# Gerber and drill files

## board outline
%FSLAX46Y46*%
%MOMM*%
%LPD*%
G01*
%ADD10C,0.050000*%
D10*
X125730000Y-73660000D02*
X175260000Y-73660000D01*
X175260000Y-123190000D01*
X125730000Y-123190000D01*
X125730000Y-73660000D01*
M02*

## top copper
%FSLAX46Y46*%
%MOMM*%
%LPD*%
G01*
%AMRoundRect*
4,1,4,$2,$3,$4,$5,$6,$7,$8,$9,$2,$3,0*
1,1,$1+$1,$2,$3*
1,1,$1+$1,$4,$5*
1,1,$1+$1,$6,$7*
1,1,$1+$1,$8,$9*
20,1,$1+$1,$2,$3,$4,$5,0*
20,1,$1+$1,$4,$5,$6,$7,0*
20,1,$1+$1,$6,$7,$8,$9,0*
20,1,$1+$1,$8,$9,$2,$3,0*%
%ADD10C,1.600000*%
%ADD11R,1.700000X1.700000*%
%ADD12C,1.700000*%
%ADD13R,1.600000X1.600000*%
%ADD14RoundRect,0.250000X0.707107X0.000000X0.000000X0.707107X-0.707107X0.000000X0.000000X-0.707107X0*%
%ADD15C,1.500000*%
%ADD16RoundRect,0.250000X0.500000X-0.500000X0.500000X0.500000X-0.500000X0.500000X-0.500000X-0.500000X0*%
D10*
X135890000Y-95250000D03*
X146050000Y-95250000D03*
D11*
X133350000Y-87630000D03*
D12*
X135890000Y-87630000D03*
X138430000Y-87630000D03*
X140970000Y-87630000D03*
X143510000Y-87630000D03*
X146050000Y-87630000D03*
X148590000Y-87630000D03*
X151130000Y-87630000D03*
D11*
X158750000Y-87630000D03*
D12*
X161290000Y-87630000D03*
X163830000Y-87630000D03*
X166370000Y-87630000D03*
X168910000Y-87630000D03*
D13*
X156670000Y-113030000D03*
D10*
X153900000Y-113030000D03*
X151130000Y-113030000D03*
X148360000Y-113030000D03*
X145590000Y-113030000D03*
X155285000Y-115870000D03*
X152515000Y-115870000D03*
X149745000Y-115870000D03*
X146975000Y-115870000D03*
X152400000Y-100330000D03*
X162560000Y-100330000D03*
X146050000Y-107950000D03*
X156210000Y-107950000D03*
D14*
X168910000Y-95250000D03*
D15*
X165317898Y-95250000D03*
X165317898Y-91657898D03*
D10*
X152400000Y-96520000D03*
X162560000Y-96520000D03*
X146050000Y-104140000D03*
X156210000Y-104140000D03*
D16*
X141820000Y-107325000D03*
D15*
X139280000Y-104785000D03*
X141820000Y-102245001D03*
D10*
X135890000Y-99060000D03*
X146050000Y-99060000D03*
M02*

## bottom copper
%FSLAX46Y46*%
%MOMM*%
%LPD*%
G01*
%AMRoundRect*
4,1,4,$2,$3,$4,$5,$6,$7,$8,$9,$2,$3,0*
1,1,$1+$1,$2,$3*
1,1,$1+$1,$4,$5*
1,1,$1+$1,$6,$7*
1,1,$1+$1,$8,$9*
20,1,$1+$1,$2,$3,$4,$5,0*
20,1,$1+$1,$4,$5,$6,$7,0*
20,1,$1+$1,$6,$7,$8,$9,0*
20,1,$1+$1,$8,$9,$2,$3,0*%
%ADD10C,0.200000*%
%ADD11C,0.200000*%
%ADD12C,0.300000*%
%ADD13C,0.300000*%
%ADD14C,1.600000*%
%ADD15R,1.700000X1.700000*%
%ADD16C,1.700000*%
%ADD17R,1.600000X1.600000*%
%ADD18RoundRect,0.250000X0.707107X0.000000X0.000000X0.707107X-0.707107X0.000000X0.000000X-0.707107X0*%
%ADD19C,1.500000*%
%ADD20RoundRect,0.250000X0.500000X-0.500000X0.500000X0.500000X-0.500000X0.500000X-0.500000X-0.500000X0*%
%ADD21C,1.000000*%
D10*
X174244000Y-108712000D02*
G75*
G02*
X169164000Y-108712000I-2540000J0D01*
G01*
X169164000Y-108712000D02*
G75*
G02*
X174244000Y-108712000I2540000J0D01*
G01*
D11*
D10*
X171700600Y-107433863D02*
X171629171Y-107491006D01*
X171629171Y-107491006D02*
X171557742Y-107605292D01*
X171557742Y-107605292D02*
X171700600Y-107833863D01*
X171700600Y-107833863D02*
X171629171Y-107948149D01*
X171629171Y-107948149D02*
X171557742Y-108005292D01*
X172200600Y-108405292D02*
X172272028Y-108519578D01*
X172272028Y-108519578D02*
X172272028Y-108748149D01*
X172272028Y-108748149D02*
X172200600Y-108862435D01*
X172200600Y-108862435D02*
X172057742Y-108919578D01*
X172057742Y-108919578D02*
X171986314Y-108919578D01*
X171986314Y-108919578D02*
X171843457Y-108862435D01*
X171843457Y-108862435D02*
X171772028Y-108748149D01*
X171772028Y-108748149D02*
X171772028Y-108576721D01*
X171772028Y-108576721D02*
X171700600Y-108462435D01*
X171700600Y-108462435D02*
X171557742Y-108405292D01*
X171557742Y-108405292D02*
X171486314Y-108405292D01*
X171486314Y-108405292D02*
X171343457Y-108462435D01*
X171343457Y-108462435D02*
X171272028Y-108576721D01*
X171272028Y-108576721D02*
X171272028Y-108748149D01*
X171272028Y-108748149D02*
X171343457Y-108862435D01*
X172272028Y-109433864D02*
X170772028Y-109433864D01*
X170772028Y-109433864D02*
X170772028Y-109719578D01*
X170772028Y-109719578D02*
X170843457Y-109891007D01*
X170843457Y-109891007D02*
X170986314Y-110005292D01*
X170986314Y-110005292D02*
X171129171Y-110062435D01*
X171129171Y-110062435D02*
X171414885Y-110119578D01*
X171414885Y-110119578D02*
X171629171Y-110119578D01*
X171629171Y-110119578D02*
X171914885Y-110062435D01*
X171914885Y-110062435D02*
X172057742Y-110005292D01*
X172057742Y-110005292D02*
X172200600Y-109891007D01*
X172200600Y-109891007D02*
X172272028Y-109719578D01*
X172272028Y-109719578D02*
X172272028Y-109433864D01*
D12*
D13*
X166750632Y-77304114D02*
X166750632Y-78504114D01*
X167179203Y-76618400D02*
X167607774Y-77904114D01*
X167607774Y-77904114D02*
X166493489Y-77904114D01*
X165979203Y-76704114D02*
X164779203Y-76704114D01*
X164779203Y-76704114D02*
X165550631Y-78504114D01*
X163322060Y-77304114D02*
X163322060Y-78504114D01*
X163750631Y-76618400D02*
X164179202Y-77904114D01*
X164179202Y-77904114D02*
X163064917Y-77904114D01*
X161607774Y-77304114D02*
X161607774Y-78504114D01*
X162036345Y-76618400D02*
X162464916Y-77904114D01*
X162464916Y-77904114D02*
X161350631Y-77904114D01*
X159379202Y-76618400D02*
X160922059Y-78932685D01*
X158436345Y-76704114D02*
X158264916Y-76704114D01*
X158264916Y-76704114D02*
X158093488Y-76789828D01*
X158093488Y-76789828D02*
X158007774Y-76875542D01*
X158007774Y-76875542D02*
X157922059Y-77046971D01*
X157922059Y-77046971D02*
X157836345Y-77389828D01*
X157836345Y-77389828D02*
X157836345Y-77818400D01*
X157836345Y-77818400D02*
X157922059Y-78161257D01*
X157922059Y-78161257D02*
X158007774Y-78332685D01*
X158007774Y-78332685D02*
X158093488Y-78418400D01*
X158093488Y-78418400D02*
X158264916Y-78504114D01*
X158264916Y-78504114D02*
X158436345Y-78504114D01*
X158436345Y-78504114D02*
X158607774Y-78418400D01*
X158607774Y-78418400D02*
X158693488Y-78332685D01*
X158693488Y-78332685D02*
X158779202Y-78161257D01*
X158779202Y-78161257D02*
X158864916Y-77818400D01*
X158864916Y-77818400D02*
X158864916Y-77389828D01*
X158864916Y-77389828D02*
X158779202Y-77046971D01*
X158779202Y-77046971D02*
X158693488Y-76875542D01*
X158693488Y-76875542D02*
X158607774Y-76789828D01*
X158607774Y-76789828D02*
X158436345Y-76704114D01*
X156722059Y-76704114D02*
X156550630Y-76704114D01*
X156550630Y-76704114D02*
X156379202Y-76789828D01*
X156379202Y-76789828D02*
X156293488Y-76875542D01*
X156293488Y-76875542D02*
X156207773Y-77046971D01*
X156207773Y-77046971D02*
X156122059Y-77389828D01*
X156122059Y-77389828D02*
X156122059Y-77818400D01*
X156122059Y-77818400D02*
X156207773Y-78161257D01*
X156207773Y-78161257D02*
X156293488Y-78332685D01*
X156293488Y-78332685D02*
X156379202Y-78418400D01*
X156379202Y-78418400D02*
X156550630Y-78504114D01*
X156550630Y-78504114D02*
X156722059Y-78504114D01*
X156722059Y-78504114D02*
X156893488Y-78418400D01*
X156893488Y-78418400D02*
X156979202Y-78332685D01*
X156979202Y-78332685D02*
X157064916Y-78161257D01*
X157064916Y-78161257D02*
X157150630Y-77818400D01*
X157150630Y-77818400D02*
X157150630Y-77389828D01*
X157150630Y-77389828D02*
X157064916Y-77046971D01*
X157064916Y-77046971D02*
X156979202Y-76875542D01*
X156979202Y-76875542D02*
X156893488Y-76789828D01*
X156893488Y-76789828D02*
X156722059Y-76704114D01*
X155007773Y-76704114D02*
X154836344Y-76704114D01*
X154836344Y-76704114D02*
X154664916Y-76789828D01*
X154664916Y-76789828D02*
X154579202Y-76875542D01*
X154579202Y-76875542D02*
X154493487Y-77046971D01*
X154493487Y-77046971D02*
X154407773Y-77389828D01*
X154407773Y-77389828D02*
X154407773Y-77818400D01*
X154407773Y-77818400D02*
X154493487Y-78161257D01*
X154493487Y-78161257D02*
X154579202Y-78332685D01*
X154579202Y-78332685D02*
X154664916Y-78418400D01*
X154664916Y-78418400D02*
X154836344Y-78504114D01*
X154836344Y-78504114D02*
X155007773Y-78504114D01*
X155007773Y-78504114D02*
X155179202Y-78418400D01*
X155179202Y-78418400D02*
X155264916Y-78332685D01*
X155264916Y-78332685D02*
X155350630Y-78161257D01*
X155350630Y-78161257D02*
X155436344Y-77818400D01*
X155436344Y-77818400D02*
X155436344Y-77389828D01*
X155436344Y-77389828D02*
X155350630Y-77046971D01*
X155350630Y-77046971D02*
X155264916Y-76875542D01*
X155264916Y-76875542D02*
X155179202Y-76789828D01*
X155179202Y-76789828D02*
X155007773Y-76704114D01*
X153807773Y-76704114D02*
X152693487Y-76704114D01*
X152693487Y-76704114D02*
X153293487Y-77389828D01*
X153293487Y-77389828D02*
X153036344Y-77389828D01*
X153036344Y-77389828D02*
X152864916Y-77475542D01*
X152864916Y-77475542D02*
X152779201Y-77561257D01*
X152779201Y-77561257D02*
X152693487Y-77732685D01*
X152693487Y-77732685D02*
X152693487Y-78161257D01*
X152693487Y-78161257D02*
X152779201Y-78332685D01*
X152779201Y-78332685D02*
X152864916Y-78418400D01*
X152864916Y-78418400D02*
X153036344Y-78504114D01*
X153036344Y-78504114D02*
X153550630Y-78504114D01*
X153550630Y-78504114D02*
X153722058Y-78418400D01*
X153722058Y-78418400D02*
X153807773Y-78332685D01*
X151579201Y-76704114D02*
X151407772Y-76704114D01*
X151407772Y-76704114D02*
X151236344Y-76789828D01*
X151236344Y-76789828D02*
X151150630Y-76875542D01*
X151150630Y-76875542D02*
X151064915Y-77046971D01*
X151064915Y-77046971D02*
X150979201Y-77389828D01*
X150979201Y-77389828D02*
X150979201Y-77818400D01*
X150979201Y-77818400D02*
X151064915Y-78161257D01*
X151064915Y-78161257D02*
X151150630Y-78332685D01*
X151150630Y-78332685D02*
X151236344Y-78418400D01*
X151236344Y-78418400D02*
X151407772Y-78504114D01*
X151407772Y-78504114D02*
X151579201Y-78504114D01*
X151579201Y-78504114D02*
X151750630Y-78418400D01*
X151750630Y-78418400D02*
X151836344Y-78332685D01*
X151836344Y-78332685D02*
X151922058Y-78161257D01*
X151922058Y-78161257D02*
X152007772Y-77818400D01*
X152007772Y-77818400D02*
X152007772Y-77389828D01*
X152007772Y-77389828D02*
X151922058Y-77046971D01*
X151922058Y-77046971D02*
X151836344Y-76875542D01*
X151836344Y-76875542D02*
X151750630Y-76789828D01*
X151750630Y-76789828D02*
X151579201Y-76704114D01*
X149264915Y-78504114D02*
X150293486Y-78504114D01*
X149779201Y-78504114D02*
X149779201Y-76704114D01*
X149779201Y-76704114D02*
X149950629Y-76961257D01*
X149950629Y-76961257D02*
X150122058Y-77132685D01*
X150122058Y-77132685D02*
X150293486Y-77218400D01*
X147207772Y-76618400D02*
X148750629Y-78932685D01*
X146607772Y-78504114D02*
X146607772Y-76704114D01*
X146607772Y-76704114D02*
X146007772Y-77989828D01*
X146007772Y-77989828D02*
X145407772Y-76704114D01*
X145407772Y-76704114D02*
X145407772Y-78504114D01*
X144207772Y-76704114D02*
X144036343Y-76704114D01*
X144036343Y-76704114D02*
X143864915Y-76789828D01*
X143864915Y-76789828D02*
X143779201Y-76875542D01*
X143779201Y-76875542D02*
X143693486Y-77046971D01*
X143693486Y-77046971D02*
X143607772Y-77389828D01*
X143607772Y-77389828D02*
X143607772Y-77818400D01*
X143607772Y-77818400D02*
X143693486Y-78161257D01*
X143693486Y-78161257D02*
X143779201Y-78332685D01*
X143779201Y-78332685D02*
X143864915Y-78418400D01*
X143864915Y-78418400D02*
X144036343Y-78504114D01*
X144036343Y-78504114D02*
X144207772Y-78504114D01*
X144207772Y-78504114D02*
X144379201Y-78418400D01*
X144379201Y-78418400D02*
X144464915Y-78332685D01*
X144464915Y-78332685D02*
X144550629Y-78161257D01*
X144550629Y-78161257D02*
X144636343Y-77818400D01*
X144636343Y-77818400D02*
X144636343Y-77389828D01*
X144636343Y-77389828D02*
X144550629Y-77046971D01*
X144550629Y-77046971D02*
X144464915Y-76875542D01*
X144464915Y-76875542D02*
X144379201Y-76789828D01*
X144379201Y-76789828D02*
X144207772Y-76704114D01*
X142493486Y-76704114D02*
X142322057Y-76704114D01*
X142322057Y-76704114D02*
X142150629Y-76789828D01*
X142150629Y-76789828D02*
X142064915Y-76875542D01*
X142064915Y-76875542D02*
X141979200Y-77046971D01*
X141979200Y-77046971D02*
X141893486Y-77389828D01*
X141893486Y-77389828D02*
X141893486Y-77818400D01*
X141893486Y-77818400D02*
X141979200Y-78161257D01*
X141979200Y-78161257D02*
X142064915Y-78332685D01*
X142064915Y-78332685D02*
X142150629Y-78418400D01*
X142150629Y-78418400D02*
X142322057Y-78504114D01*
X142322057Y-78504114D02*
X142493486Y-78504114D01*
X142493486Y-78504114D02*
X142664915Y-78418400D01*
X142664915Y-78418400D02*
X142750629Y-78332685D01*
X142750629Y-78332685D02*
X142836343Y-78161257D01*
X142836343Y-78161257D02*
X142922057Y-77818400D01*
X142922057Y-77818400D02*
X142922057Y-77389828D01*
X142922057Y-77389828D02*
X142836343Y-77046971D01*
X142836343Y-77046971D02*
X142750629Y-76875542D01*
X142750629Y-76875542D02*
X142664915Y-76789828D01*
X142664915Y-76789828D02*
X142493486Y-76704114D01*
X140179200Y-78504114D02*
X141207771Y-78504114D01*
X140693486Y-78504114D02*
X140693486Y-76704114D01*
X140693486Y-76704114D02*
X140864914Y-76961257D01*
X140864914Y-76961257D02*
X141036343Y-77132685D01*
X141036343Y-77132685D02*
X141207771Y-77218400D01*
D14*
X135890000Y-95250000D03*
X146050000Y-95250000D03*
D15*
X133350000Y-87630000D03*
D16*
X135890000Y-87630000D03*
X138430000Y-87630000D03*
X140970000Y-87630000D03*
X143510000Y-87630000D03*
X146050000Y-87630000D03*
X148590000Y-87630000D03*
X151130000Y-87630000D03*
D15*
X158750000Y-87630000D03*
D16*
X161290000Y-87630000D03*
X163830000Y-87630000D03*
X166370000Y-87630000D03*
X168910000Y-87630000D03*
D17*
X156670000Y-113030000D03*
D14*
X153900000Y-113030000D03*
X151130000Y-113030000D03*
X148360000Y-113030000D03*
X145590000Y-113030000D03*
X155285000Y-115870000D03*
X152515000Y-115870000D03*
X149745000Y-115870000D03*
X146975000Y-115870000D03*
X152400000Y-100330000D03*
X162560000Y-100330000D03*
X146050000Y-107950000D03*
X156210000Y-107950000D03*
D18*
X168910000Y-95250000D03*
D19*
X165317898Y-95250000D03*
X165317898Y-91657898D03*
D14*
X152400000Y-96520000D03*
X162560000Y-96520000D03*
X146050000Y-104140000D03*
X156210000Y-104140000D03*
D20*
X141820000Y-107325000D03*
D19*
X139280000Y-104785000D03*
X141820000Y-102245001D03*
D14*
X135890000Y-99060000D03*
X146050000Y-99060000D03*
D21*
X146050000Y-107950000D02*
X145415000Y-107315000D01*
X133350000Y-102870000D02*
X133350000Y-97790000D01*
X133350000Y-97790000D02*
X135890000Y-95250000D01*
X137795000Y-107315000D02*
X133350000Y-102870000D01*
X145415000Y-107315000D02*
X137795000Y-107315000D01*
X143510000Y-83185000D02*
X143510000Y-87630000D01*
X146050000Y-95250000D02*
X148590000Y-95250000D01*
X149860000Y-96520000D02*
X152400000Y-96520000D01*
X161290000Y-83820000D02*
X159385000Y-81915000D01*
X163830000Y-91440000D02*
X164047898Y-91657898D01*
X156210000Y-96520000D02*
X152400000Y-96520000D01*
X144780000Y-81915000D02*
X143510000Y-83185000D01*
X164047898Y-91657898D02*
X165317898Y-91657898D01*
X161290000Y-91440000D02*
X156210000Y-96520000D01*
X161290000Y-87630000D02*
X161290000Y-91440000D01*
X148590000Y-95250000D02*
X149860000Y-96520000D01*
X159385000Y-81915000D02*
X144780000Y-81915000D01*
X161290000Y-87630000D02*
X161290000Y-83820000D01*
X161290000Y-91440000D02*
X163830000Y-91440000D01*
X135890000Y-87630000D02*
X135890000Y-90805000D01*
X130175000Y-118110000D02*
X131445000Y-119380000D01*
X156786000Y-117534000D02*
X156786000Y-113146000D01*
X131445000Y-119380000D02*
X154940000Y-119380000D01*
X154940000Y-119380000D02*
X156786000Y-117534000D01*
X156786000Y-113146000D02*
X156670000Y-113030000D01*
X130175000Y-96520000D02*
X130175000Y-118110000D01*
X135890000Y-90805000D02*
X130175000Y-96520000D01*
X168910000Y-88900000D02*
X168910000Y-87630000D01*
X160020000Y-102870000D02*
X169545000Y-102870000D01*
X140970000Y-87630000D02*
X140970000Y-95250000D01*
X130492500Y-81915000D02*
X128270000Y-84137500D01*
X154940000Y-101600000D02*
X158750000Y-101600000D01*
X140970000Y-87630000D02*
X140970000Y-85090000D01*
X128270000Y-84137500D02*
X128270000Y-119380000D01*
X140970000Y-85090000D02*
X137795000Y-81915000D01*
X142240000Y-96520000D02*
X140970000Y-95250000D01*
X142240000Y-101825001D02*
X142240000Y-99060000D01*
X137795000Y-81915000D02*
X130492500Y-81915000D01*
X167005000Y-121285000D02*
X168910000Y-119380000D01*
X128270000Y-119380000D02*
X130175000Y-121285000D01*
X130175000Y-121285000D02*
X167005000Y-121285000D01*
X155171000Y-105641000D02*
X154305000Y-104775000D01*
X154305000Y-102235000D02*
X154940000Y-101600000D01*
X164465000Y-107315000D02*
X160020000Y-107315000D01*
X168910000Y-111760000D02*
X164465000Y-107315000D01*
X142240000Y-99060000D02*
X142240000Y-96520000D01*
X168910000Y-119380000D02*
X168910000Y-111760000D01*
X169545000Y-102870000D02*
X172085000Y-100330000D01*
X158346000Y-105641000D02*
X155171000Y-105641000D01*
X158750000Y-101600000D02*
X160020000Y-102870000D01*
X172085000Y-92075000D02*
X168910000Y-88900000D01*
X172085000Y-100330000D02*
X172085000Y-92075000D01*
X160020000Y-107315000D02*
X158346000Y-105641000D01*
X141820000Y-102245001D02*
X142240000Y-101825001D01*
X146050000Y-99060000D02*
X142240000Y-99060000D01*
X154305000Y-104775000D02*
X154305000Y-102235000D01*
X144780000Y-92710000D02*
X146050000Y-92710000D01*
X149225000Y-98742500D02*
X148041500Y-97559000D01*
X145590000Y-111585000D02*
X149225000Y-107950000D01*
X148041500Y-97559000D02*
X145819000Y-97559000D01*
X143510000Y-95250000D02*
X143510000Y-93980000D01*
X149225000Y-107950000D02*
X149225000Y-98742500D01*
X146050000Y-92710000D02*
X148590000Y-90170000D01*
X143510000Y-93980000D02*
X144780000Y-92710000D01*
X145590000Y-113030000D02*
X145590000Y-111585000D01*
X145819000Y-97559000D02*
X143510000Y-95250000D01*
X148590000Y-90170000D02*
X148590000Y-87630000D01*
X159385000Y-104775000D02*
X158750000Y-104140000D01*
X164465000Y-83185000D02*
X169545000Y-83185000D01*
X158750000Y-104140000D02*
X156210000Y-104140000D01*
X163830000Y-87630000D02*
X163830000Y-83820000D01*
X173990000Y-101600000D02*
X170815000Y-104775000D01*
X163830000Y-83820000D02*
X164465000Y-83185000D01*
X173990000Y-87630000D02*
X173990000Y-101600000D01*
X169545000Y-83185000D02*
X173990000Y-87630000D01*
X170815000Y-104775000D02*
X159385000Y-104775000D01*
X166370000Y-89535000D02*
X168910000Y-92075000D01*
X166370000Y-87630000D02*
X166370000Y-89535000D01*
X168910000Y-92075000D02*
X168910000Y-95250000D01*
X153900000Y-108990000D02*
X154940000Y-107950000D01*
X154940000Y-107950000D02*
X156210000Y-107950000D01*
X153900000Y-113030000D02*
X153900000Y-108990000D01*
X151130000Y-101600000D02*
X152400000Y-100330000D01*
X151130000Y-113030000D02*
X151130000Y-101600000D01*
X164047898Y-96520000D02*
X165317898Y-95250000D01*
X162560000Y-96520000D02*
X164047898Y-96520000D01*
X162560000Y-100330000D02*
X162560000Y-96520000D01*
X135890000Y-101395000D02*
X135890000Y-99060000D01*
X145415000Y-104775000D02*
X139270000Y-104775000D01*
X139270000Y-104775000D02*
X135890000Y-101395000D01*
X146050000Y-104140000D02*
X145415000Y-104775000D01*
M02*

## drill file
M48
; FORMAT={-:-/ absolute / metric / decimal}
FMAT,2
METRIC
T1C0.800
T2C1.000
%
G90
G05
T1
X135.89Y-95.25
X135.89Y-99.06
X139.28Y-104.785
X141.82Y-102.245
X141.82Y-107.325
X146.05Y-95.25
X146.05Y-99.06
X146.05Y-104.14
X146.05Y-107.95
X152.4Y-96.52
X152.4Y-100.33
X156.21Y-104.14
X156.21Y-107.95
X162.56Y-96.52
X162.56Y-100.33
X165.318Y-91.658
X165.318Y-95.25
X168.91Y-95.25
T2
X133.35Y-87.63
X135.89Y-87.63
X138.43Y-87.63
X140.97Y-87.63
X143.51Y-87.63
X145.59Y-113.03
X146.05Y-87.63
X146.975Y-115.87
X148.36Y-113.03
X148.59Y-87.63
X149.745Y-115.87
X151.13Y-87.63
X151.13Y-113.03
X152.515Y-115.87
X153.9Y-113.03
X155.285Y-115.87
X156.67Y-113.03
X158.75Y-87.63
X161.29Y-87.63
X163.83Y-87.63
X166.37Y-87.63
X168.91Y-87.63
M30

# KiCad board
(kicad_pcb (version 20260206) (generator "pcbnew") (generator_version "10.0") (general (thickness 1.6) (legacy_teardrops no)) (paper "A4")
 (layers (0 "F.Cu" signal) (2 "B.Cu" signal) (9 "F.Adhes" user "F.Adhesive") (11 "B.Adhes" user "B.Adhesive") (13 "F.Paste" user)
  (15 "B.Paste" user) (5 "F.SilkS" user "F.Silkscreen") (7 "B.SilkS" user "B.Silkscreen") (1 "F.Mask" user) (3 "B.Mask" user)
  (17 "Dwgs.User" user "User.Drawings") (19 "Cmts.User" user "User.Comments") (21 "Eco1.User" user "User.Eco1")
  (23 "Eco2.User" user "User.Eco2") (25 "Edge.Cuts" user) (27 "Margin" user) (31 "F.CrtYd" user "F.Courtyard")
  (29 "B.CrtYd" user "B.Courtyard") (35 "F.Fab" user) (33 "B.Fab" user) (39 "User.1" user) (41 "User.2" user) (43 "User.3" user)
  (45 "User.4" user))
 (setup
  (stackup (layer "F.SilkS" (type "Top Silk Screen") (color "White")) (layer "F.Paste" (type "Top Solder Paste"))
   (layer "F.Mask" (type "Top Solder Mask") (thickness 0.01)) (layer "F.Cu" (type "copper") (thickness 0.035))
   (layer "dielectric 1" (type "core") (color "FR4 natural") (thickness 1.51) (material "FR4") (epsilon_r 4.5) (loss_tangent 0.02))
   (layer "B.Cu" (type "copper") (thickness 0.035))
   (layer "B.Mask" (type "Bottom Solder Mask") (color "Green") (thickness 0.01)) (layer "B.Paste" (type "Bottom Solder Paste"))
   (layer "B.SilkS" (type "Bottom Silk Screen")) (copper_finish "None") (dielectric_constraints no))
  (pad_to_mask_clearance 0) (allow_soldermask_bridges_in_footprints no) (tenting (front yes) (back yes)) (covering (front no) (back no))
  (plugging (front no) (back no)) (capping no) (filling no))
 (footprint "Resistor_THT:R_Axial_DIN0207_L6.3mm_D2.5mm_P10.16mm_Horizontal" (layer "F.Cu") (at 135.89 95.25)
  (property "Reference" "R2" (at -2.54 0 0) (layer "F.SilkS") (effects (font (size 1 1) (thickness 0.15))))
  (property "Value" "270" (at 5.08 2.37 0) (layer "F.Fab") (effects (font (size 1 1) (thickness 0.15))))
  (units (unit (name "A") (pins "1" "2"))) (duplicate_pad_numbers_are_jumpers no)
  (pad "1" thru_hole circle (at 0 0) (size 1.6 1.6) (drill 0.8) (layers "*.Cu" "*.Mask") (remove_unused_layers no) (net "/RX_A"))
  (pad "2" thru_hole circle (at 10.16 0) (size 1.6 1.6) (drill 0.8) (layers "*.Cu" "*.Mask") (remove_unused_layers no) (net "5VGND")))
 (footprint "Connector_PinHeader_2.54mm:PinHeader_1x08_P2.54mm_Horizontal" (layer "F.Cu") (at 133.35 87.63 90)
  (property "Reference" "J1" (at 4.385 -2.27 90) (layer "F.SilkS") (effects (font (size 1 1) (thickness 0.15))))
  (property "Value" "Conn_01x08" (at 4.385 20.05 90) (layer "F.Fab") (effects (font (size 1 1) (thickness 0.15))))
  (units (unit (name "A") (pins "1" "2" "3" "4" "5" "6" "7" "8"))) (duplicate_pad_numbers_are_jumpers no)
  (pad "1" thru_hole rect (at 0 0 90) (size 1.7 1.7) (drill 1) (layers "*.Cu" "*.Mask") (remove_unused_layers no) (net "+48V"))
  (pad "2" thru_hole circle (at 0 2.54 90) (size 1.7 1.7) (drill 1) (layers "*.Cu" "*.Mask") (remove_unused_layers no)
   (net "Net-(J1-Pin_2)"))
  (pad "3" thru_hole circle (at 0 5.08 90) (size 1.7 1.7) (drill 1) (layers "*.Cu" "*.Mask") (remove_unused_layers no) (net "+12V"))
  (pad "4" thru_hole circle (at 0 7.62 90) (size 1.7 1.7) (drill 1) (layers "*.Cu" "*.Mask") (remove_unused_layers no) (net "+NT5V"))
  (pad "5" thru_hole circle (at 0 10.16 90) (size 1.7 1.7) (drill 1) (layers "*.Cu" "*.Mask") (remove_unused_layers no) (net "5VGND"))
  (pad "6" thru_hole circle (at 0 12.7 90) (size 1.7 1.7) (drill 1) (layers "*.Cu" "*.Mask") (remove_unused_layers no) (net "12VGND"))
  (pad "7" thru_hole circle (at 0 15.24 90) (size 1.7 1.7) (drill 1) (layers "*.Cu" "*.Mask") (remove_unused_layers no) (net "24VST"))
  (pad "8" thru_hole circle (at 0 17.78 90) (size 1.7 1.7) (drill 1) (layers "*.Cu" "*.Mask") (remove_unused_layers no)
   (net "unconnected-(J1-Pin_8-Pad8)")))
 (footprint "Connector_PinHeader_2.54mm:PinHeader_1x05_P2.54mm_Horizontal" (layer "F.Cu") (at 158.75 87.63 90)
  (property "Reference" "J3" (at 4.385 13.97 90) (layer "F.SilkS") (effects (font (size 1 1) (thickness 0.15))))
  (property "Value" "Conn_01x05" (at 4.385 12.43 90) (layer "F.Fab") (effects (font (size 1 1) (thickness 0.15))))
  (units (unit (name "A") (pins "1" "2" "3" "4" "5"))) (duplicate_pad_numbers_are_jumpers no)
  (pad "1" thru_hole rect (at 0 0 90) (size 1.7 1.7) (drill 1) (layers "*.Cu" "*.Mask") (remove_unused_layers no)
   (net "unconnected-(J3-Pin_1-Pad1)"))
  (pad "2" thru_hole circle (at 0 2.54 90) (size 1.7 1.7) (drill 1) (layers "*.Cu" "*.Mask") (remove_unused_layers no) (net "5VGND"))
  (pad "3" thru_hole circle (at 0 5.08 90) (size 1.7 1.7) (drill 1) (layers "*.Cu" "*.Mask") (remove_unused_layers no) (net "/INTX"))
  (pad "4" thru_hole circle (at 0 7.62 90) (size 1.7 1.7) (drill 1) (layers "*.Cu" "*.Mask") (remove_unused_layers no) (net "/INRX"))
  (pad "5" thru_hole circle (at 0 10.16 90) (size 1.7 1.7) (drill 1) (layers "*.Cu" "*.Mask") (remove_unused_layers no) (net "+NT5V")))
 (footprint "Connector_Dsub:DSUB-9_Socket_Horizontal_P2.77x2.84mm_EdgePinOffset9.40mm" (layer "F.Cu") (at 156.67 113.03)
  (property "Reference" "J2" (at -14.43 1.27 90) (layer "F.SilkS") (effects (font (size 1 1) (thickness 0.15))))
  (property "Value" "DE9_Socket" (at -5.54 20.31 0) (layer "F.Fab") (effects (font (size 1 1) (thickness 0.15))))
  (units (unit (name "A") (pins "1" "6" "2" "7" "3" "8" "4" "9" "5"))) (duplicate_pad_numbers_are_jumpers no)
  (pad "1" thru_hole rect (at 0 0) (size 1.6 1.6) (drill 1) (layers "*.Cu" "*.Mask") (remove_unused_layers no) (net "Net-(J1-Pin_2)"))
  (pad "2" thru_hole circle (at -2.77 0) (size 1.6 1.6) (drill 1) (layers "*.Cu" "*.Mask") (remove_unused_layers no) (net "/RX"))
  (pad "3" thru_hole circle (at -5.54 0) (size 1.6 1.6) (drill 1) (layers "*.Cu" "*.Mask") (remove_unused_layers no) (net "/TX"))
  (pad "4" thru_hole circle (at -8.31 0) (size 1.6 1.6) (drill 1) (layers "*.Cu" "*.Mask") (remove_unused_layers no)
   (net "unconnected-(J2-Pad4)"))
  (pad "5" thru_hole circle (at -11.08 0) (size 1.6 1.6) (drill 1) (layers "*.Cu" "*.Mask") (remove_unused_layers no) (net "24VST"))
  (pad "6" thru_hole circle (at -1.385 2.84) (size 1.6 1.6) (drill 1) (layers "*.Cu" "*.Mask") (remove_unused_layers no)
   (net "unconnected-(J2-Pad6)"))
  (pad "7" thru_hole circle (at -4.155 2.84) (size 1.6 1.6) (drill 1) (layers "*.Cu" "*.Mask") (remove_unused_layers no)
   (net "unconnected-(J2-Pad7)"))
  (pad "8" thru_hole circle (at -6.925 2.84) (size 1.6 1.6) (drill 1) (layers "*.Cu" "*.Mask") (remove_unused_layers no)
   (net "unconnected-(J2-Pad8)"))
  (pad "9" thru_hole circle (at -9.695 2.84) (size 1.6 1.6) (drill 1) (layers "*.Cu" "*.Mask") (remove_unused_layers no)
   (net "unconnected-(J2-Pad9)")))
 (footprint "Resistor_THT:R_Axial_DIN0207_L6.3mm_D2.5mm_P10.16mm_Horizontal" (layer "F.Cu") (at 152.4 100.33)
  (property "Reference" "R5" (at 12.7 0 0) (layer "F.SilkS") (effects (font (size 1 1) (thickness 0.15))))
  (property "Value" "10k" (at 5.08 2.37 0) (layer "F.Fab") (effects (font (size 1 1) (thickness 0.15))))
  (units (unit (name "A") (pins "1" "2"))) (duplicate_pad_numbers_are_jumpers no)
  (pad "1" thru_hole circle (at 0 0) (size 1.6 1.6) (drill 0.8) (layers "*.Cu" "*.Mask") (remove_unused_layers no) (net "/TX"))
  (pad "2" thru_hole circle (at 10.16 0) (size 1.6 1.6) (drill 0.8) (layers "*.Cu" "*.Mask") (remove_unused_layers no) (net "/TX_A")))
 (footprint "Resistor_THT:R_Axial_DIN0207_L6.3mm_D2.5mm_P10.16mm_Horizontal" (layer "F.Cu") (at 146.05 107.95)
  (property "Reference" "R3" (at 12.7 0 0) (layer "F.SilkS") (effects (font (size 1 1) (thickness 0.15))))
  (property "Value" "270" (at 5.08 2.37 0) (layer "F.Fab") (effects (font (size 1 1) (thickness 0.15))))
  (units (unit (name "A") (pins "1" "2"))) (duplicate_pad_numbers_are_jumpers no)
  (pad "1" thru_hole circle (at 0 0) (size 1.6 1.6) (drill 0.8) (layers "*.Cu" "*.Mask") (remove_unused_layers no) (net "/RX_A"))
  (pad "2" thru_hole circle (at 10.16 0) (size 1.6 1.6) (drill 0.8) (layers "*.Cu" "*.Mask") (remove_unused_layers no) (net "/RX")))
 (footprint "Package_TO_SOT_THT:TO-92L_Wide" (layer "F.Cu") (at 168.91 95.25 135)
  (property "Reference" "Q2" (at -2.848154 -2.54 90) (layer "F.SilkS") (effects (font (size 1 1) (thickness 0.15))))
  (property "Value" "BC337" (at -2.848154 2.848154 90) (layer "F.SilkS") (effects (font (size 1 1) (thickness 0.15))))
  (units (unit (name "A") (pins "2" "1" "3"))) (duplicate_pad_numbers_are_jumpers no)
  (pad "1" thru_hole roundrect (at 0 0 135) (size 1.5 1.5) (drill 0.8) (layers "*.Cu" "*.Mask") (remove_unused_layers no)
   (roundrect_rratio 0.1666666667) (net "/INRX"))
  (pad "2" thru_hole circle (at 2.54 -2.54 135) (size 1.5 1.5) (drill 0.8) (layers "*.Cu" "*.Mask") (remove_unused_layers no) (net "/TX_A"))
  (pad "3" thru_hole circle (at 5.079999 0 135) (size 1.5 1.5) (drill 0.8) (layers "*.Cu" "*.Mask") (remove_unused_layers no) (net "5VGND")))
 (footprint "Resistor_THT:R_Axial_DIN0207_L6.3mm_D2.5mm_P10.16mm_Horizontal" (layer "F.Cu") (at 152.4 96.52)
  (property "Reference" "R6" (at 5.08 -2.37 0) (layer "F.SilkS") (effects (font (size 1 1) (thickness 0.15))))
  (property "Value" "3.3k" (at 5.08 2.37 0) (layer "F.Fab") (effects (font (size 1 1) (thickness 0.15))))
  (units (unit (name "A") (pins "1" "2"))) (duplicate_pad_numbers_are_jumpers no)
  (pad "1" thru_hole circle (at 0 0) (size 1.6 1.6) (drill 0.8) (layers "*.Cu" "*.Mask") (remove_unused_layers no) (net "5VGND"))
  (pad "2" thru_hole circle (at 10.16 0) (size 1.6 1.6) (drill 0.8) (layers "*.Cu" "*.Mask") (remove_unused_layers no) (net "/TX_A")))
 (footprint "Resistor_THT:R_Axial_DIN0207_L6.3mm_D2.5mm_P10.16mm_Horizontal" (layer "F.Cu") (at 146.05 104.14)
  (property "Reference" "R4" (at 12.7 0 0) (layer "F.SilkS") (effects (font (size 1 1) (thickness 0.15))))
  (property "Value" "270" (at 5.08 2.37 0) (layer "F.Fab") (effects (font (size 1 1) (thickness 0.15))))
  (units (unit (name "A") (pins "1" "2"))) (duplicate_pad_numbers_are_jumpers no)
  (pad "1" thru_hole circle (at 0 0) (size 1.6 1.6) (drill 0.8) (layers "*.Cu" "*.Mask") (remove_unused_layers no) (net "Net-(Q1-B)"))
  (pad "2" thru_hole circle (at 10.16 0) (size 1.6 1.6) (drill 0.8) (layers "*.Cu" "*.Mask") (remove_unused_layers no) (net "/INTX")))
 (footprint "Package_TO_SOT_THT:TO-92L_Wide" (layer "F.Cu") (at 141.82 107.325 90)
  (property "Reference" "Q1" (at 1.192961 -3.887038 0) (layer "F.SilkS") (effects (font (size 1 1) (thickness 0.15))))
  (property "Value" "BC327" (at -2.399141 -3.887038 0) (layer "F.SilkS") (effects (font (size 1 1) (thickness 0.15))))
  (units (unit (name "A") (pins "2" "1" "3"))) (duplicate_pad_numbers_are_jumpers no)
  (pad "1" thru_hole roundrect (at 0 0 90) (size 1.5 1.5) (drill 0.8) (layers "*.Cu" "*.Mask") (remove_unused_layers no)
   (roundrect_rratio 0.1666666667) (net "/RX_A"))
  (pad "2" thru_hole circle (at 2.54 -2.54 90) (size 1.5 1.5) (drill 0.8) (layers "*.Cu" "*.Mask") (remove_unused_layers no)
   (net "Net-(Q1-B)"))
  (pad "3" thru_hole circle (at 5.079999 0 90) (size 1.5 1.5) (drill 0.8) (layers "*.Cu" "*.Mask") (remove_unused_layers no) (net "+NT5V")))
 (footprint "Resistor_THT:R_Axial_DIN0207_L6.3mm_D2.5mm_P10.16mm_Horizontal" (layer "F.Cu") (at 135.89 99.06)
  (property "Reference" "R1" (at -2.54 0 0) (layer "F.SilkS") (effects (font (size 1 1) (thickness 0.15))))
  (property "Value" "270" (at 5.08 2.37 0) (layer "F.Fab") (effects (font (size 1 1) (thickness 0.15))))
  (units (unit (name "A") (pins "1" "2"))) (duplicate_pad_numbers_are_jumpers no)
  (pad "1" thru_hole circle (at 0 0) (size 1.6 1.6) (drill 0.8) (layers "*.Cu" "*.Mask") (remove_unused_layers no) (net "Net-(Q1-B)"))
  (pad "2" thru_hole circle (at 10.16 0) (size 1.6 1.6) (drill 0.8) (layers "*.Cu" "*.Mask") (remove_unused_layers no) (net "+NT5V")))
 (gr_circle (center 171.704 108.712) (end 174.244 108.712) (stroke (width 0.2) (type default)) (fill no) (layer "B.Cu"))
 (gr_rect (start 125.73 73.66) (end 175.26 123.19) (stroke (width 0.05) (type default)) (fill no) (layer "Edge.Cuts"))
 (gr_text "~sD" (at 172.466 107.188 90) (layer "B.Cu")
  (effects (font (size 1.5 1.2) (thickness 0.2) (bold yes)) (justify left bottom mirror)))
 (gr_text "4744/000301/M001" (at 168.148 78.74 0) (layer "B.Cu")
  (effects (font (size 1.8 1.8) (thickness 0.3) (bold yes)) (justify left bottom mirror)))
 (segment (start 146.05 107.95) (end 145.415 107.315) (width 1) (layer "B.Cu") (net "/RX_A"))
 (segment (start 133.35 102.87) (end 133.35 97.79) (width 1) (layer "B.Cu") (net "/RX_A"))
 (segment (start 133.35 97.79) (end 135.89 95.25) (width 1) (layer "B.Cu") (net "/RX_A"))
 (segment (start 137.795 107.315) (end 133.35 102.87) (width 1) (layer "B.Cu") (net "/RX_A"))
 (segment (start 145.415 107.315) (end 137.795 107.315) (width 1) (layer "B.Cu") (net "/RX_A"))
 (segment (start 143.51 83.185) (end 143.51 87.63) (width 1) (layer "B.Cu") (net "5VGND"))
 (segment (start 146.05 95.25) (end 148.59 95.25) (width 1) (layer "B.Cu") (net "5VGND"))
 (segment (start 149.86 96.52) (end 152.4 96.52) (width 1) (layer "B.Cu") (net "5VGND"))
 (segment (start 161.29 83.82) (end 159.385 81.915) (width 1) (layer "B.Cu") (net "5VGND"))
 (segment (start 163.83 91.44) (end 164.047898 91.657898) (width 1) (layer "B.Cu") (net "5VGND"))
 (segment (start 156.21 96.52) (end 152.4 96.52) (width 1) (layer "B.Cu") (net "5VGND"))
 (segment (start 144.78 81.915) (end 143.51 83.185) (width 1) (layer "B.Cu") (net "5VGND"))
 (segment (start 164.047898 91.657898) (end 165.317898 91.657898) (width 1) (layer "B.Cu") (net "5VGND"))
 (segment (start 161.29 91.44) (end 156.21 96.52) (width 1) (layer "B.Cu") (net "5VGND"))
 (segment (start 161.29 87.63) (end 161.29 91.44) (width 1) (layer "B.Cu") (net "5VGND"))
 (segment (start 148.59 95.25) (end 149.86 96.52) (width 1) (layer "B.Cu") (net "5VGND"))
 (segment (start 159.385 81.915) (end 144.78 81.915) (width 1) (layer "B.Cu") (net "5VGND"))
 (segment (start 161.29 87.63) (end 161.29 83.82) (width 1) (layer "B.Cu") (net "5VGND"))
 (segment (start 161.29 91.44) (end 163.83 91.44) (width 1) (layer "B.Cu") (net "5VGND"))
 (segment (start 135.89 87.63) (end 135.89 90.805) (width 1) (layer "B.Cu") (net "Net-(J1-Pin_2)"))
 (segment (start 130.175 118.11) (end 131.445 119.38) (width 1) (layer "B.Cu") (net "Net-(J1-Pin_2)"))
 (segment (start 156.786 117.534) (end 156.786 113.146) (width 1) (layer "B.Cu") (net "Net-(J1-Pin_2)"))
 (segment (start 131.445 119.38) (end 154.94 119.38) (width 1) (layer "B.Cu") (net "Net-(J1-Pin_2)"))
 (segment (start 154.94 119.38) (end 156.786 117.534) (width 1) (layer "B.Cu") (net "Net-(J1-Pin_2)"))
 (segment (start 156.786 113.146) (end 156.67 113.03) (width 1) (layer "B.Cu") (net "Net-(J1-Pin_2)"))
 (segment (start 130.175 96.52) (end 130.175 118.11) (width 1) (layer "B.Cu") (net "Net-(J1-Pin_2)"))
 (segment (start 135.89 90.805) (end 130.175 96.52) (width 1) (layer "B.Cu") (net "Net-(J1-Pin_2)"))
 (segment (start 168.91 88.9) (end 168.91 87.63) (width 1) (layer "B.Cu") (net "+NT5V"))
 (segment (start 160.02 102.87) (end 169.545 102.87) (width 1) (layer "B.Cu") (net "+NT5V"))
 (segment (start 140.97 87.63) (end 140.97 95.25) (width 1) (layer "B.Cu") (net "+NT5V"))
 (segment (start 130.4925 81.915) (end 128.27 84.1375) (width 1) (layer "B.Cu") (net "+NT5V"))
 (segment (start 154.94 101.6) (end 158.75 101.6) (width 1) (layer "B.Cu") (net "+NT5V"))
 (segment (start 140.97 87.63) (end 140.97 85.09) (width 1) (layer "B.Cu") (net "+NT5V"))
 (segment (start 128.27 84.1375) (end 128.27 119.38) (width 1) (layer "B.Cu") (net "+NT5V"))
 (segment (start 140.97 85.09) (end 137.795 81.915) (width 1) (layer "B.Cu") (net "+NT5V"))
 (segment (start 142.24 96.52) (end 140.97 95.25) (width 1) (layer "B.Cu") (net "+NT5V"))
 (segment (start 142.24 101.825001) (end 142.24 99.06) (width 1) (layer "B.Cu") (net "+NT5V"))
 (segment (start 137.795 81.915) (end 130.4925 81.915) (width 1) (layer "B.Cu") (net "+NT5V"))
 (segment (start 167.005 121.285) (end 168.91 119.38) (width 1) (layer "B.Cu") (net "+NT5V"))
 (segment (start 128.27 119.38) (end 130.175 121.285) (width 1) (layer "B.Cu") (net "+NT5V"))
 (segment (start 130.175 121.285) (end 167.005 121.285) (width 1) (layer "B.Cu") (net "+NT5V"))
 (segment (start 155.171 105.641) (end 154.305 104.775) (width 1) (layer "B.Cu") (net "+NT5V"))
 (segment (start 154.305 102.235) (end 154.94 101.6) (width 1) (layer "B.Cu") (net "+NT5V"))
 (segment (start 164.465 107.315) (end 160.02 107.315) (width 1) (layer "B.Cu") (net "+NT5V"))
 (segment (start 168.91 111.76) (end 164.465 107.315) (width 1) (layer "B.Cu") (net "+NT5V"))
 (segment (start 142.24 99.06) (end 142.24 96.52) (width 1) (layer "B.Cu") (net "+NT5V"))
 (segment (start 168.91 119.38) (end 168.91 111.76) (width 1) (layer "B.Cu") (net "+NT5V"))
 (segment (start 169.545 102.87) (end 172.085 100.33) (width 1) (layer "B.Cu") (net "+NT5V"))
 (segment (start 158.346 105.641) (end 155.171 105.641) (width 1) (layer "B.Cu") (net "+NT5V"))
 (segment (start 158.75 101.6) (end 160.02 102.87) (width 1) (layer "B.Cu") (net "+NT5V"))
 (segment (start 172.085 92.075) (end 168.91 88.9) (width 1) (layer "B.Cu") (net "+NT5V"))
 (segment (start 172.085 100.33) (end 172.085 92.075) (width 1) (layer "B.Cu") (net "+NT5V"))
 (segment (start 160.02 107.315) (end 158.346 105.641) (width 1) (layer "B.Cu") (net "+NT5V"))
 (segment (start 141.82 102.245001) (end 142.24 101.825001) (width 1) (layer "B.Cu") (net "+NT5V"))
 (segment (start 146.05 99.06) (end 142.24 99.06) (width 1) (layer "B.Cu") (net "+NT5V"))
 (segment (start 154.305 104.775) (end 154.305 102.235) (width 1) (layer "B.Cu") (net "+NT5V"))
 (segment (start 144.78 92.71) (end 146.05 92.71) (width 1) (layer "B.Cu") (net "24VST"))
 (segment (start 149.225 98.7425) (end 148.0415 97.559) (width 1) (layer "B.Cu") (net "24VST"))
 (segment (start 145.59 111.585) (end 149.225 107.95) (width 1) (layer "B.Cu") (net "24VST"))
 (segment (start 148.0415 97.559) (end 145.819 97.559) (width 1) (layer "B.Cu") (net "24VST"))
 (segment (start 143.51 95.25) (end 143.51 93.98) (width 1) (layer "B.Cu") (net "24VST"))
 (segment (start 149.225 107.95) (end 149.225 98.7425) (width 1) (layer "B.Cu") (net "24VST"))
 (segment (start 146.05 92.71) (end 148.59 90.17) (width 1) (layer "B.Cu") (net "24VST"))
 (segment (start 143.51 93.98) (end 144.78 92.71) (width 1) (layer "B.Cu") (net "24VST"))
 (segment (start 145.59 113.03) (end 145.59 111.585) (width 1) (layer "B.Cu") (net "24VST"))
 (segment (start 145.819 97.559) (end 143.51 95.25) (width 1) (layer "B.Cu") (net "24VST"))
 (segment (start 148.59 90.17) (end 148.59 87.63) (width 1) (layer "B.Cu") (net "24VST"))
 (segment (start 159.385 104.775) (end 158.75 104.14) (width 1) (layer "B.Cu") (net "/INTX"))
 (segment (start 164.465 83.185) (end 169.545 83.185) (width 1) (layer "B.Cu") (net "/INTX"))
 (segment (start 158.75 104.14) (end 156.21 104.14) (width 1) (layer "B.Cu") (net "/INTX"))
 (segment (start 163.83 87.63) (end 163.83 83.82) (width 1) (layer "B.Cu") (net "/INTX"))
 (segment (start 173.99 101.6) (end 170.815 104.775) (width 1) (layer "B.Cu") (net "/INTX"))
 (segment (start 163.83 83.82) (end 164.465 83.185) (width 1) (layer "B.Cu") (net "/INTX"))
 (segment (start 173.99 87.63) (end 173.99 101.6) (width 1) (layer "B.Cu") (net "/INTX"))
 (segment (start 169.545 83.185) (end 173.99 87.63) (width 1) (layer "B.Cu") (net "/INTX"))
 (segment (start 170.815 104.775) (end 159.385 104.775) (width 1) (layer "B.Cu") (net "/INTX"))
 (segment (start 166.37 89.535) (end 168.91 92.075) (width 1) (layer "B.Cu") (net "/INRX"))
 (segment (start 166.37 87.63) (end 166.37 89.535) (width 1) (layer "B.Cu") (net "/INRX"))
 (segment (start 168.91 92.075) (end 168.91 95.25) (width 1) (layer "B.Cu") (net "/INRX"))
 (segment (start 153.9 108.99) (end 154.94 107.95) (width 1) (layer "B.Cu") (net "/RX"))
 (segment (start 154.94 107.95) (end 156.21 107.95) (width 1) (layer "B.Cu") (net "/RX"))
 (segment (start 153.9 113.03) (end 153.9 108.99) (width 1) (layer "B.Cu") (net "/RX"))
 (segment (start 151.13 101.6) (end 152.4 100.33) (width 1) (layer "B.Cu") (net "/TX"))
 (segment (start 151.13 113.03) (end 151.13 101.6) (width 1) (layer "B.Cu") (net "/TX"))
 (segment (start 164.047898 96.52) (end 165.317898 95.25) (width 1) (layer "B.Cu") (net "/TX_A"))
 (segment (start 162.56 96.52) (end 164.047898 96.52) (width 1) (layer "B.Cu") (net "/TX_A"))
 (segment (start 162.56 100.33) (end 162.56 96.52) (width 1) (layer "B.Cu") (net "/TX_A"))
 (segment (start 135.89 101.395) (end 135.89 99.06) (width 1) (layer "B.Cu") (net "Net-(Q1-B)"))
 (segment (start 145.415 104.775) (end 139.27 104.775) (width 1) (layer "B.Cu") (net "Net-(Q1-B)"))
 (segment (start 139.27 104.775) (end 135.89 101.395) (width 1) (layer "B.Cu") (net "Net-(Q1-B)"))
 (segment (start 146.05 104.14) (end 145.415 104.775) (width 1) (layer "B.Cu") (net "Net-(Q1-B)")))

